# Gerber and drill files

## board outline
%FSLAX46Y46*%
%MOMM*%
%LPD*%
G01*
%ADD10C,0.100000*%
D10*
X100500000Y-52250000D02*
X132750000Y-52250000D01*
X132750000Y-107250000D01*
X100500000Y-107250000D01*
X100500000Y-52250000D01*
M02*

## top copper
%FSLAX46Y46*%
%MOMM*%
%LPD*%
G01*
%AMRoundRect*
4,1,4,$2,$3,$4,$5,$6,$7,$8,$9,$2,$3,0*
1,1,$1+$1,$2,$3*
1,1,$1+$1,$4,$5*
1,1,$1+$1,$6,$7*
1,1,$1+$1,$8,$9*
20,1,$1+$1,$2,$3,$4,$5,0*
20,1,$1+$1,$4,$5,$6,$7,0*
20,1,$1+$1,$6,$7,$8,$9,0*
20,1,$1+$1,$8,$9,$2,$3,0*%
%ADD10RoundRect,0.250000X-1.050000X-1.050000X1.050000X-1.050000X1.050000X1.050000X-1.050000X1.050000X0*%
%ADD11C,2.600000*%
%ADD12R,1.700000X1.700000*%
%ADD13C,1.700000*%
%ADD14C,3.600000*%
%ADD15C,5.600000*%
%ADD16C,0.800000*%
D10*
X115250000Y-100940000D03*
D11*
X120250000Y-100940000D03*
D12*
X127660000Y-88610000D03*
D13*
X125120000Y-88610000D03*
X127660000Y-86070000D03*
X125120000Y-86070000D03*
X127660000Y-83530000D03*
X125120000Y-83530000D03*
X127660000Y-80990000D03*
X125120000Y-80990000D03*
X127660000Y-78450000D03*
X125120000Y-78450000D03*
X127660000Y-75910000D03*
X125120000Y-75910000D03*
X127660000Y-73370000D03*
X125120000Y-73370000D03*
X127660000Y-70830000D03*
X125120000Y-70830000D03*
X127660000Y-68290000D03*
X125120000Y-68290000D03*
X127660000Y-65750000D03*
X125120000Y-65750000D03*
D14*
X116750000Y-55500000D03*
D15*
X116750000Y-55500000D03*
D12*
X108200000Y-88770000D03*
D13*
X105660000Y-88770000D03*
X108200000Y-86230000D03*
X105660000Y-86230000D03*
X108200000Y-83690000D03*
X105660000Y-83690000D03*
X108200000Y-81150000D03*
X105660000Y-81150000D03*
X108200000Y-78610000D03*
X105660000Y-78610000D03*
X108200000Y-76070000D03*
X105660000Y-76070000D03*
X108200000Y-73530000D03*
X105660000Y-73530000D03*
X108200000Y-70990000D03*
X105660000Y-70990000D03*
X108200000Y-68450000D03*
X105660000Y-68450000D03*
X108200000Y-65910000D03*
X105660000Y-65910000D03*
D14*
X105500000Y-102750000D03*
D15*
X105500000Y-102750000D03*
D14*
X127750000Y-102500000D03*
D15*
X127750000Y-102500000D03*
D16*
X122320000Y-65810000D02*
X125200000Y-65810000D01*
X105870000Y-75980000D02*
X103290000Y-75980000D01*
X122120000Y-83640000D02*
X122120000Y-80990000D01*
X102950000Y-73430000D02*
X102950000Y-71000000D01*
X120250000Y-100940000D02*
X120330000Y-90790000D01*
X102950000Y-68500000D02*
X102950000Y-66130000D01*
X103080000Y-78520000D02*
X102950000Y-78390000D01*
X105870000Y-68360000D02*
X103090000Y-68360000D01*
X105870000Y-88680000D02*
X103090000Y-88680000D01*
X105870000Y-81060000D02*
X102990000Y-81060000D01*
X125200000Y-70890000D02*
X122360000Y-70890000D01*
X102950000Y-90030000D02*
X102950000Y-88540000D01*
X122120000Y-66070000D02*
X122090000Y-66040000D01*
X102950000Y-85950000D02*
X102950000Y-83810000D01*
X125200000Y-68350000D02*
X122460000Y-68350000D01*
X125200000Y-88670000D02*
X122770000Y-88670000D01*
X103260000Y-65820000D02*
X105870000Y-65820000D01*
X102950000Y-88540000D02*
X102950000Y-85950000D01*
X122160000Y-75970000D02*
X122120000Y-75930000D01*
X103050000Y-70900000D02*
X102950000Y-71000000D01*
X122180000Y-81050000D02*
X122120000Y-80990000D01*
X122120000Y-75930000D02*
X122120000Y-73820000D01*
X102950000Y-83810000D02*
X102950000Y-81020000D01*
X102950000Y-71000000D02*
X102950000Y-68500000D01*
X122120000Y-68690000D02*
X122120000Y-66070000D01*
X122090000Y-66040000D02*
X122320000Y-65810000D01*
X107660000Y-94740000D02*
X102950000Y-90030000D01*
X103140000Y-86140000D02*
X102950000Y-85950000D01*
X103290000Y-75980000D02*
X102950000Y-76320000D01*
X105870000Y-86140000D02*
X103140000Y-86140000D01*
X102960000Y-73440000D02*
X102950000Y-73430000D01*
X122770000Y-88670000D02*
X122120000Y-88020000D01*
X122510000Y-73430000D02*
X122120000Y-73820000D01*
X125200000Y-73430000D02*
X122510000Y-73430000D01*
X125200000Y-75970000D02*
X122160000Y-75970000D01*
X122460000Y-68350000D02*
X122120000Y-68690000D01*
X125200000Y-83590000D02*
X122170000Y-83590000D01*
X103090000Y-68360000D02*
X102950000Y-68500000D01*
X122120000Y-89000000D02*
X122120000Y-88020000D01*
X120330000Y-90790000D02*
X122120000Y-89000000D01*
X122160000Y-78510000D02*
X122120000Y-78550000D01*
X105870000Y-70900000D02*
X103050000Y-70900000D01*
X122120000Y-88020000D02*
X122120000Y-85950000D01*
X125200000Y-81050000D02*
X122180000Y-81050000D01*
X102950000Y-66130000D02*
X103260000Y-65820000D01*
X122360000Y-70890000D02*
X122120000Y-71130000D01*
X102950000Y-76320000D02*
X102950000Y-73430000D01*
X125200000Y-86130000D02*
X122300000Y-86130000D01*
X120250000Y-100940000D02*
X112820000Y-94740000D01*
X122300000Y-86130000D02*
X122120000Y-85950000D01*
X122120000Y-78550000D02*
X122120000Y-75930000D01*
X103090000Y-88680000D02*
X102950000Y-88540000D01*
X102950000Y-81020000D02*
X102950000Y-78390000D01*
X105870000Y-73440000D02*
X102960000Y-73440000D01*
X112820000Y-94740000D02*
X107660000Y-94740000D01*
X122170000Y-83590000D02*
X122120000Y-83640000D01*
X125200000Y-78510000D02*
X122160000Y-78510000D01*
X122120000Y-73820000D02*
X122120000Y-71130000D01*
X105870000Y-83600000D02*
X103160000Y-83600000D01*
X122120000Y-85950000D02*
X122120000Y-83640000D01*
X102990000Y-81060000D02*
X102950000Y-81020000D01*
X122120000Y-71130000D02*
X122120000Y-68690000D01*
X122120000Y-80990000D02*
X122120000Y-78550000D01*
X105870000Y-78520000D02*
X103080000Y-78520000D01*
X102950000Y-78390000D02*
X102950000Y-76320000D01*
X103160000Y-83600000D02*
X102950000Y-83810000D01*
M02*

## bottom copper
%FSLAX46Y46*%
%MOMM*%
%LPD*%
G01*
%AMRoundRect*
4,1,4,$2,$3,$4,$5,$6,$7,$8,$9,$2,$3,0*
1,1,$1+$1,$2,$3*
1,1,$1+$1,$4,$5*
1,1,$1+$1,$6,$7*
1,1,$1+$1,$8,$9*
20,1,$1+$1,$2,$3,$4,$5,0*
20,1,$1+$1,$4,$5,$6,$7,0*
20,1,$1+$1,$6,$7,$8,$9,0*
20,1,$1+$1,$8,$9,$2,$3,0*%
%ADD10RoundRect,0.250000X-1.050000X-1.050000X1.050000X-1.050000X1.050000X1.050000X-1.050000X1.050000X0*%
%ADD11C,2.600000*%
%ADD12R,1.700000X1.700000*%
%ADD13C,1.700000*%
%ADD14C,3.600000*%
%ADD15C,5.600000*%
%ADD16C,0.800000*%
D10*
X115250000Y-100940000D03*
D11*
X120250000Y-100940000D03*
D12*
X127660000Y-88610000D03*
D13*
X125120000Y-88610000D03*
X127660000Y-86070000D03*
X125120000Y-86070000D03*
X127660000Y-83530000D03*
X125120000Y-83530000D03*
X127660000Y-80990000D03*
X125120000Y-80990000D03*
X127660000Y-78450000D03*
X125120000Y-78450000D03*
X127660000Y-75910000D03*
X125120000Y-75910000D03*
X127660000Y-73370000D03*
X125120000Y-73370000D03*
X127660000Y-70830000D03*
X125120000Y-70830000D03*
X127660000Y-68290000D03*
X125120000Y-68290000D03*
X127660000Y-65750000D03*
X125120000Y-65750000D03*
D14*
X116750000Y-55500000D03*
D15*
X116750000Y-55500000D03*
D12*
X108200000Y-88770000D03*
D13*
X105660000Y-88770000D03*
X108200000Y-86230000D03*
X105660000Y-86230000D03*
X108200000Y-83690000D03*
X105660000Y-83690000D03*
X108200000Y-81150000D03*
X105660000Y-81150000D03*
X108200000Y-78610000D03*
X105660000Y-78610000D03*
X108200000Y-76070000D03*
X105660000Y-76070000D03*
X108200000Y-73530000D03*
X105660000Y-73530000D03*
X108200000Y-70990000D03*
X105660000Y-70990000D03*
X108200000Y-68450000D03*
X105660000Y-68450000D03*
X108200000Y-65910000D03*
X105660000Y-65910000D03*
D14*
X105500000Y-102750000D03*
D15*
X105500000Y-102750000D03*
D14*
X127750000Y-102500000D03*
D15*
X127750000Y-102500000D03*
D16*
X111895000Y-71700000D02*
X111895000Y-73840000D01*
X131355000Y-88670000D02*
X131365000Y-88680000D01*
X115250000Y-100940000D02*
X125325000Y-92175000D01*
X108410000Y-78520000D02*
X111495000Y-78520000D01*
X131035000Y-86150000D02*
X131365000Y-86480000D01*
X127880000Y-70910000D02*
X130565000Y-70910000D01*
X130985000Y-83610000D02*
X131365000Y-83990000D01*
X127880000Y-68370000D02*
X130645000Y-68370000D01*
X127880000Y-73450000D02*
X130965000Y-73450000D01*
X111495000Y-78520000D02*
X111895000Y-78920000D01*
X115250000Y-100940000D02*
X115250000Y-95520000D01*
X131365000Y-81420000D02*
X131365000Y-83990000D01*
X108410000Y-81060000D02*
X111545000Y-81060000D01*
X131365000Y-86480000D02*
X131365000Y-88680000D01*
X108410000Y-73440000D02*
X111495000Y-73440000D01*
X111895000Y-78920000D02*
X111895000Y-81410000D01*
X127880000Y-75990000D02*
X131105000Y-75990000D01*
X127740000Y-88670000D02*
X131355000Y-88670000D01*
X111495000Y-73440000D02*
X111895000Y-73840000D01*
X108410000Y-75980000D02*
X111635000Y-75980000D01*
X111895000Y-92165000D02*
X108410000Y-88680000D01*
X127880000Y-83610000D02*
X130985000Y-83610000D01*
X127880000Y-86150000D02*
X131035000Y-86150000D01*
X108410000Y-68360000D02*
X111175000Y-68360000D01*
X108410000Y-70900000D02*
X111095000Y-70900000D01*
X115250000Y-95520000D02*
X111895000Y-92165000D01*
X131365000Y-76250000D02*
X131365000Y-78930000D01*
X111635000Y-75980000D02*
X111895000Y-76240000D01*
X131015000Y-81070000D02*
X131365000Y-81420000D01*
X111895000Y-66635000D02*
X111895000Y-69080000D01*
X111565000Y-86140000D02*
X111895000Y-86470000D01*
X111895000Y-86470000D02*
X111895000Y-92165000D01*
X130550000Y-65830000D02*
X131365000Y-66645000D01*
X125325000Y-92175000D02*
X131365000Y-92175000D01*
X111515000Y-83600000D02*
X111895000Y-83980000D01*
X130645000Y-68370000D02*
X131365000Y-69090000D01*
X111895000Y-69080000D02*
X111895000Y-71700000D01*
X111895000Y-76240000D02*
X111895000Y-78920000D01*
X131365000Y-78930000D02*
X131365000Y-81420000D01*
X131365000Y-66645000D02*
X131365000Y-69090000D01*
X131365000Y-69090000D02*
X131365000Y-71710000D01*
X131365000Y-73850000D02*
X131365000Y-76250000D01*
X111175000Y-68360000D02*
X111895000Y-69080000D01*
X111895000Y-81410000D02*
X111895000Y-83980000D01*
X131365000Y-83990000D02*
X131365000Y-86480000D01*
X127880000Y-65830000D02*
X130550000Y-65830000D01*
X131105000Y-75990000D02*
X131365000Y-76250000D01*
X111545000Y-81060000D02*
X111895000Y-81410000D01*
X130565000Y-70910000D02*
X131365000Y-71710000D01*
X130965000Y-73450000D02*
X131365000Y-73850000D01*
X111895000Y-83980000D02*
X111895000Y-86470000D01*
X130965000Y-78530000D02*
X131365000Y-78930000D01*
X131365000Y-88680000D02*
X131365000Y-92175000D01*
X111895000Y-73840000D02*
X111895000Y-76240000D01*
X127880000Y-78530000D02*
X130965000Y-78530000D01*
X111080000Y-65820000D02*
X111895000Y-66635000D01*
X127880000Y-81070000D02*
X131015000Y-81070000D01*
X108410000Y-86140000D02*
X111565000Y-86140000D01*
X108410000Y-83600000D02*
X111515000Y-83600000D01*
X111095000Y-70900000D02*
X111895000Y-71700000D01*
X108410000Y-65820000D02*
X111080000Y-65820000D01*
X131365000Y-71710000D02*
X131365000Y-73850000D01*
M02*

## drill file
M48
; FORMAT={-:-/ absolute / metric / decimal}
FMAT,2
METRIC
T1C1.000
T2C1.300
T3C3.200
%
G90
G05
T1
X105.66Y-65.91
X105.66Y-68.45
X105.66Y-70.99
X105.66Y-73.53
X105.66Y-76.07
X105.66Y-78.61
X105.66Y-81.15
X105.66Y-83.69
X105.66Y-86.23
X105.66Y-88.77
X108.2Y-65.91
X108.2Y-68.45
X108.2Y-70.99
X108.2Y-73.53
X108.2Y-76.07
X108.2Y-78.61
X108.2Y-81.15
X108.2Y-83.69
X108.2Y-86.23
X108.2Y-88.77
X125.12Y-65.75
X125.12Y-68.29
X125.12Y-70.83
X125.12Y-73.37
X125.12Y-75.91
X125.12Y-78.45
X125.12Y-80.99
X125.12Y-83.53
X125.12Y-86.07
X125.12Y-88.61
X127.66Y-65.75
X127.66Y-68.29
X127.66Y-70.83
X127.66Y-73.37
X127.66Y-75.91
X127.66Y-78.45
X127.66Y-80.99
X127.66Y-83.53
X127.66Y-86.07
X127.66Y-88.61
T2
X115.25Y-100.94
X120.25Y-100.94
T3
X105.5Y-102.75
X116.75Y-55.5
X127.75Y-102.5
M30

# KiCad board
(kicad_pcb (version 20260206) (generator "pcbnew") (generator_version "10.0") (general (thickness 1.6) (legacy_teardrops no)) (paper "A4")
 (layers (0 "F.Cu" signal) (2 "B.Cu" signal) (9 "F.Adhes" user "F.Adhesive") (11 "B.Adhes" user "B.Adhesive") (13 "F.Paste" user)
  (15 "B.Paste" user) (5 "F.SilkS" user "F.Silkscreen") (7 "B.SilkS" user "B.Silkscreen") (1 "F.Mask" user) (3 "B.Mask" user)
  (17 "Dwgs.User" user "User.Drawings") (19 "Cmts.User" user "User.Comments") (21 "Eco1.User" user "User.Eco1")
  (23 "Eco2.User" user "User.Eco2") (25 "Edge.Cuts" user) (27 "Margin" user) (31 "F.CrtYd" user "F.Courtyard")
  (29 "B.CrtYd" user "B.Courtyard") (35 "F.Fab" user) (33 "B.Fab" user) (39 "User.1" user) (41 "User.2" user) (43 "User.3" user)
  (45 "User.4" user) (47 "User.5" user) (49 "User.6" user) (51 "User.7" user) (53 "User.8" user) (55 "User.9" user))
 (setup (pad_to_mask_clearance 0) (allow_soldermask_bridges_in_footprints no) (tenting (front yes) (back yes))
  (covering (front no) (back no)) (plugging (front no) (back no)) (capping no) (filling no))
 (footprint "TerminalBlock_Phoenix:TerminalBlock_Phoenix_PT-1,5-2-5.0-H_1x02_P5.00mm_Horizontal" (layer "F.Cu") (at 115.25 100.94)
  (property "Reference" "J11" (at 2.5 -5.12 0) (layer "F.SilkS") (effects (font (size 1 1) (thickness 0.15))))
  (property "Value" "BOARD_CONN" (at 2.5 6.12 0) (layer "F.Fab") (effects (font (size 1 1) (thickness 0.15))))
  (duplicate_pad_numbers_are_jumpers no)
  (pad "1" thru_hole roundrect (at 0 0) (size 2.6 2.6) (drill 1.3) (layers "*.Cu" "*.Mask") (remove_unused_layers no)
   (roundrect_rratio 0.096154) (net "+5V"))
  (pad "2" thru_hole circle (at 5 0) (size 2.6 2.6) (drill 1.3) (layers "*.Cu" "*.Mask") (remove_unused_layers no) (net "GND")))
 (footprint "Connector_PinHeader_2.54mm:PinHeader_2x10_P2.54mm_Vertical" (layer "F.Cu") (at 127.66 88.61 180)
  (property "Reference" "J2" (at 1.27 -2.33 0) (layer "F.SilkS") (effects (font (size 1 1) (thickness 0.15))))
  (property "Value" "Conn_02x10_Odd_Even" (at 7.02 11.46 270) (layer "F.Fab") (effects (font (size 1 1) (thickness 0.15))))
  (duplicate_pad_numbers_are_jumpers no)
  (pad "1" thru_hole rect (at 0 0 180) (size 1.7 1.7) (drill 1) (layers "*.Cu" "*.Mask") (remove_unused_layers no) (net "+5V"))
  (pad "2" thru_hole circle (at 2.54 0 180) (size 1.7 1.7) (drill 1) (layers "*.Cu" "*.Mask") (remove_unused_layers no) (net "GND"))
  (pad "3" thru_hole circle (at 0 2.54 180) (size 1.7 1.7) (drill 1) (layers "*.Cu" "*.Mask") (remove_unused_layers no) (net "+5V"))
  (pad "4" thru_hole circle (at 2.54 2.54 180) (size 1.7 1.7) (drill 1) (layers "*.Cu" "*.Mask") (remove_unused_layers no) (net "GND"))
  (pad "5" thru_hole circle (at 0 5.08 180) (size 1.7 1.7) (drill 1) (layers "*.Cu" "*.Mask") (remove_unused_layers no) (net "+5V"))
  (pad "6" thru_hole circle (at 2.54 5.08 180) (size 1.7 1.7) (drill 1) (layers "*.Cu" "*.Mask") (remove_unused_layers no) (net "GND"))
  (pad "7" thru_hole circle (at 0 7.62 180) (size 1.7 1.7) (drill 1) (layers "*.Cu" "*.Mask") (remove_unused_layers no) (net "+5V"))
  (pad "8" thru_hole circle (at 2.54 7.62 180) (size 1.7 1.7) (drill 1) (layers "*.Cu" "*.Mask") (remove_unused_layers no) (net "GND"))
  (pad "9" thru_hole circle (at 0 10.16 180) (size 1.7 1.7) (drill 1) (layers "*.Cu" "*.Mask") (remove_unused_layers no) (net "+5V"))
  (pad "10" thru_hole circle (at 2.54 10.16 180) (size 1.7 1.7) (drill 1) (layers "*.Cu" "*.Mask") (remove_unused_layers no) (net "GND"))
  (pad "11" thru_hole circle (at 0 12.7 180) (size 1.7 1.7) (drill 1) (layers "*.Cu" "*.Mask") (remove_unused_layers no) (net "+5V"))
  (pad "12" thru_hole circle (at 2.54 12.7 180) (size 1.7 1.7) (drill 1) (layers "*.Cu" "*.Mask") (remove_unused_layers no) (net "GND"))
  (pad "13" thru_hole circle (at 0 15.24 180) (size 1.7 1.7) (drill 1) (layers "*.Cu" "*.Mask") (remove_unused_layers no) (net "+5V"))
  (pad "14" thru_hole circle (at 2.54 15.24 180) (size 1.7 1.7) (drill 1) (layers "*.Cu" "*.Mask") (remove_unused_layers no) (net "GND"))
  (pad "15" thru_hole circle (at 0 17.78 180) (size 1.7 1.7) (drill 1) (layers "*.Cu" "*.Mask") (remove_unused_layers no) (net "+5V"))
  (pad "16" thru_hole circle (at 2.54 17.78 180) (size 1.7 1.7) (drill 1) (layers "*.Cu" "*.Mask") (remove_unused_layers no) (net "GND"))
  (pad "17" thru_hole circle (at 0 20.32 180) (size 1.7 1.7) (drill 1) (layers "*.Cu" "*.Mask") (remove_unused_layers no) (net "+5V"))
  (pad "18" thru_hole circle (at 2.54 20.32 180) (size 1.7 1.7) (drill 1) (layers "*.Cu" "*.Mask") (remove_unused_layers no) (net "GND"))
  (pad "19" thru_hole circle (at 0 22.86 180) (size 1.7 1.7) (drill 1) (layers "*.Cu" "*.Mask") (remove_unused_layers no) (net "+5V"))
  (pad "20" thru_hole circle (at 2.54 22.86 180) (size 1.7 1.7) (drill 1) (layers "*.Cu" "*.Mask") (remove_unused_layers no) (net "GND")))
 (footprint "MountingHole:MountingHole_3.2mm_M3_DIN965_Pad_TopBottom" (layer "F.Cu") (at 116.75 55.5)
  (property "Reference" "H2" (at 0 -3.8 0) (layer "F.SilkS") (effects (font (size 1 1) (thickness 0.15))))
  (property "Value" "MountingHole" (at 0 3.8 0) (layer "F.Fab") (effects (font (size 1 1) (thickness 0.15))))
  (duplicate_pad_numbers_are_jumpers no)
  (pad "1" thru_hole circle (at 0 0) (size 3.6 3.6) (drill 3.2) (layers "*.Cu" "*.Mask") (remove_unused_layers no) (zone_connect 2))
  (pad "1" connect circle (at 0 0) (size 5.6 5.6) (layers "F.Cu" "F.Mask") (zone_connect 2))
  (pad "1" connect circle (at 0 0) (size 5.6 5.6) (layers "B.Cu" "B.Mask") (zone_connect 2)))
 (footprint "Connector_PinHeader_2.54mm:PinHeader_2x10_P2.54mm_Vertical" (layer "F.Cu") (at 108.2 88.77 180)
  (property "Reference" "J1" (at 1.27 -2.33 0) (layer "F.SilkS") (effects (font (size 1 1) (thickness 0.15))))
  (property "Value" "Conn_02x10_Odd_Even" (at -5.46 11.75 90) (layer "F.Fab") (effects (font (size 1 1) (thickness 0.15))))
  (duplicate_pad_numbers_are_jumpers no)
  (pad "1" thru_hole rect (at 0 0 180) (size 1.7 1.7) (drill 1) (layers "*.Cu" "*.Mask") (remove_unused_layers no) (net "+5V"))
  (pad "2" thru_hole circle (at 2.54 0 180) (size 1.7 1.7) (drill 1) (layers "*.Cu" "*.Mask") (remove_unused_layers no) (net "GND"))
  (pad "3" thru_hole circle (at 0 2.54 180) (size 1.7 1.7) (drill 1) (layers "*.Cu" "*.Mask") (remove_unused_layers no) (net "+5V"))
  (pad "4" thru_hole circle (at 2.54 2.54 180) (size 1.7 1.7) (drill 1) (layers "*.Cu" "*.Mask") (remove_unused_layers no) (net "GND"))
  (pad "5" thru_hole circle (at 0 5.08 180) (size 1.7 1.7) (drill 1) (layers "*.Cu" "*.Mask") (remove_unused_layers no) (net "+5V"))
  (pad "6" thru_hole circle (at 2.54 5.08 180) (size 1.7 1.7) (drill 1) (layers "*.Cu" "*.Mask") (remove_unused_layers no) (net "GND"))
  (pad "7" thru_hole circle (at 0 7.62 180) (size 1.7 1.7) (drill 1) (layers "*.Cu" "*.Mask") (remove_unused_layers no) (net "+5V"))
  (pad "8" thru_hole circle (at 2.54 7.62 180) (size 1.7 1.7) (drill 1) (layers "*.Cu" "*.Mask") (remove_unused_layers no) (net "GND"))
  (pad "9" thru_hole circle (at 0 10.16 180) (size 1.7 1.7) (drill 1) (layers "*.Cu" "*.Mask") (remove_unused_layers no) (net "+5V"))
  (pad "10" thru_hole circle (at 2.54 10.16 180) (size 1.7 1.7) (drill 1) (layers "*.Cu" "*.Mask") (remove_unused_layers no) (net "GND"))
  (pad "11" thru_hole circle (at 0 12.7 180) (size 1.7 1.7) (drill 1) (layers "*.Cu" "*.Mask") (remove_unused_layers no) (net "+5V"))
  (pad "12" thru_hole circle (at 2.54 12.7 180) (size 1.7 1.7) (drill 1) (layers "*.Cu" "*.Mask") (remove_unused_layers no) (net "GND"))
  (pad "13" thru_hole circle (at 0 15.24 180) (size 1.7 1.7) (drill 1) (layers "*.Cu" "*.Mask") (remove_unused_layers no) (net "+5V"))
  (pad "14" thru_hole circle (at 2.54 15.24 180) (size 1.7 1.7) (drill 1) (layers "*.Cu" "*.Mask") (remove_unused_layers no) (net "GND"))
  (pad "15" thru_hole circle (at 0 17.78 180) (size 1.7 1.7) (drill 1) (layers "*.Cu" "*.Mask") (remove_unused_layers no) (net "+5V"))
  (pad "16" thru_hole circle (at 2.54 17.78 180) (size 1.7 1.7) (drill 1) (layers "*.Cu" "*.Mask") (remove_unused_layers no) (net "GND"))
  (pad "17" thru_hole circle (at 0 20.32 180) (size 1.7 1.7) (drill 1) (layers "*.Cu" "*.Mask") (remove_unused_layers no) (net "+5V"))
  (pad "18" thru_hole circle (at 2.54 20.32 180) (size 1.7 1.7) (drill 1) (layers "*.Cu" "*.Mask") (remove_unused_layers no) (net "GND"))
  (pad "19" thru_hole circle (at 0 22.86 180) (size 1.7 1.7) (drill 1) (layers "*.Cu" "*.Mask") (remove_unused_layers no) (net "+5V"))
  (pad "20" thru_hole circle (at 2.54 22.86 180) (size 1.7 1.7) (drill 1) (layers "*.Cu" "*.Mask") (remove_unused_layers no) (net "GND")))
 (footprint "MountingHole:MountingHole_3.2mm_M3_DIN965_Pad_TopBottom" (layer "F.Cu") (at 105.5 102.75)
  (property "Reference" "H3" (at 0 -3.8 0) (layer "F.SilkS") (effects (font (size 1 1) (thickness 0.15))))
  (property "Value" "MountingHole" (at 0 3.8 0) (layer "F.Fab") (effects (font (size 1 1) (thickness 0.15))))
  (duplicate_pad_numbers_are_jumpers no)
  (pad "1" thru_hole circle (at 0 0) (size 3.6 3.6) (drill 3.2) (layers "*.Cu" "*.Mask") (remove_unused_layers no) (zone_connect 2))
  (pad "1" connect circle (at 0 0) (size 5.6 5.6) (layers "F.Cu" "F.Mask") (zone_connect 2))
  (pad "1" connect circle (at 0 0) (size 5.6 5.6) (layers "B.Cu" "B.Mask") (zone_connect 2)))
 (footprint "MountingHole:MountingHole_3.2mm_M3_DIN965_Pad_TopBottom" (layer "F.Cu") (at 127.75 102.5)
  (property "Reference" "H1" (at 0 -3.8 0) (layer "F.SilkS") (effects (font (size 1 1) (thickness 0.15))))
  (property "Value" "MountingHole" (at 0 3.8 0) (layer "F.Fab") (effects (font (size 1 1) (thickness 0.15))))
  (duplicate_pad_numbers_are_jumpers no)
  (pad "1" thru_hole circle (at 0 0) (size 3.6 3.6) (drill 3.2) (layers "*.Cu" "*.Mask") (remove_unused_layers no) (zone_connect 2))
  (pad "1" connect circle (at 0 0) (size 5.6 5.6) (layers "F.Cu" "F.Mask") (zone_connect 2))
  (pad "1" connect circle (at 0 0) (size 5.6 5.6) (layers "B.Cu" "B.Mask") (zone_connect 2)))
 (gr_rect (start 100.5 52.25) (end 132.75 107.25) (stroke (width 0.1) (type default)) (fill no) (layer "Edge.Cuts"))
 (segment (start 111.895 71.7) (end 111.895 73.84) (width 0.8) (layer "B.Cu") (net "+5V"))
 (segment (start 131.355 88.67) (end 131.365 88.68) (width 0.8) (layer "B.Cu") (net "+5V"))
 (segment (start 115.25 100.94) (end 125.325 92.175) (width 0.8) (layer "B.Cu") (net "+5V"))
 (segment (start 108.41 78.52) (end 111.495 78.52) (width 0.8) (layer "B.Cu") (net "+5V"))
 (segment (start 131.035 86.15) (end 131.365 86.48) (width 0.8) (layer "B.Cu") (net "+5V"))
 (segment (start 127.88 70.91) (end 130.565 70.91) (width 0.8) (layer "B.Cu") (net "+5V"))
 (segment (start 130.985 83.61) (end 131.365 83.99) (width 0.8) (layer "B.Cu") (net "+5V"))
 (segment (start 127.88 68.37) (end 130.645 68.37) (width 0.8) (layer "B.Cu") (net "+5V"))
 (segment (start 127.88 73.45) (end 130.965 73.45) (width 0.8) (layer "B.Cu") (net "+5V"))
 (segment (start 111.495 78.52) (end 111.895 78.92) (width 0.8) (layer "B.Cu") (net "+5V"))
 (segment (start 115.25 100.94) (end 115.25 95.52) (width 0.8) (layer "B.Cu") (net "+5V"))
 (segment (start 131.365 81.42) (end 131.365 83.99) (width 0.8) (layer "B.Cu") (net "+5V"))
 (segment (start 108.41 81.06) (end 111.545 81.06) (width 0.8) (layer "B.Cu") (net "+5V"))
 (segment (start 131.365 86.48) (end 131.365 88.68) (width 0.8) (layer "B.Cu") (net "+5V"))
 (segment (start 108.41 73.44) (end 111.495 73.44) (width 0.8) (layer "B.Cu") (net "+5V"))
 (segment (start 111.895 78.92) (end 111.895 81.41) (width 0.8) (layer "B.Cu") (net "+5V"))
 (segment (start 127.88 75.99) (end 131.105 75.99) (width 0.8) (layer "B.Cu") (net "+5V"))
 (segment (start 127.74 88.67) (end 131.355 88.67) (width 0.8) (layer "B.Cu") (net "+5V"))
 (segment (start 111.495 73.44) (end 111.895 73.84) (width 0.8) (layer "B.Cu") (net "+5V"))
 (segment (start 108.41 75.98) (end 111.635 75.98) (width 0.8) (layer "B.Cu") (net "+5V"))
 (segment (start 111.895 92.165) (end 108.41 88.68) (width 0.8) (layer "B.Cu") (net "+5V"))
 (segment (start 127.88 83.61) (end 130.985 83.61) (width 0.8) (layer "B.Cu") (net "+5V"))
 (segment (start 127.88 86.15) (end 131.035 86.15) (width 0.8) (layer "B.Cu") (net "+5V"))
 (segment (start 108.41 68.36) (end 111.175 68.36) (width 0.8) (layer "B.Cu") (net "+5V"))
 (segment (start 108.41 70.9) (end 111.095 70.9) (width 0.8) (layer "B.Cu") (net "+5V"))
 (segment (start 115.25 95.52) (end 111.895 92.165) (width 0.8) (layer "B.Cu") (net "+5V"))
 (segment (start 131.365 76.25) (end 131.365 78.93) (width 0.8) (layer "B.Cu") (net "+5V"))
 (segment (start 111.635 75.98) (end 111.895 76.24) (width 0.8) (layer "B.Cu") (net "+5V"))
 (segment (start 131.015 81.07) (end 131.365 81.42) (width 0.8) (layer "B.Cu") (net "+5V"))
 (segment (start 111.895 66.635) (end 111.895 69.08) (width 0.8) (layer "B.Cu") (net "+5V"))
 (segment (start 111.565 86.14) (end 111.895 86.47) (width 0.8) (layer "B.Cu") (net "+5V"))
 (segment (start 111.895 86.47) (end 111.895 92.165) (width 0.8) (layer "B.Cu") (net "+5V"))
 (segment (start 130.55 65.83) (end 131.365 66.645) (width 0.8) (layer "B.Cu") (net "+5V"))
 (segment (start 125.325 92.175) (end 131.365 92.175) (width 0.8) (layer "B.Cu") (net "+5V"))
 (segment (start 111.515 83.6) (end 111.895 83.98) (width 0.8) (layer "B.Cu") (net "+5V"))
 (segment (start 130.645 68.37) (end 131.365 69.09) (width 0.8) (layer "B.Cu") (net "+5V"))
 (segment (start 111.895 69.08) (end 111.895 71.7) (width 0.8) (layer "B.Cu") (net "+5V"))
 (segment (start 111.895 76.24) (end 111.895 78.92) (width 0.8) (layer "B.Cu") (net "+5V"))
 (segment (start 131.365 78.93) (end 131.365 81.42) (width 0.8) (layer "B.Cu") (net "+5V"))
 (segment (start 131.365 66.645) (end 131.365 69.09) (width 0.8) (layer "B.Cu") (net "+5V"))
 (segment (start 131.365 69.09) (end 131.365 71.71) (width 0.8) (layer "B.Cu") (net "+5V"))
 (segment (start 131.365 73.85) (end 131.365 76.25) (width 0.8) (layer "B.Cu") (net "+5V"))
 (segment (start 111.175 68.36) (end 111.895 69.08) (width 0.8) (layer "B.Cu") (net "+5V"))
 (segment (start 111.895 81.41) (end 111.895 83.98) (width 0.8) (layer "B.Cu") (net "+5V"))
 (segment (start 131.365 83.99) (end 131.365 86.48) (width 0.8) (layer "B.Cu") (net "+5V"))
 (segment (start 127.88 65.83) (end 130.55 65.83) (width 0.8) (layer "B.Cu") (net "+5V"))
 (segment (start 131.105 75.99) (end 131.365 76.25) (width 0.8) (layer "B.Cu") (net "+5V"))
 (segment (start 111.545 81.06) (end 111.895 81.41) (width 0.8) (layer "B.Cu") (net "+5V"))
 (segment (start 130.565 70.91) (end 131.365 71.71) (width 0.8) (layer "B.Cu") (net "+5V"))
 (segment (start 130.965 73.45) (end 131.365 73.85) (width 0.8) (layer "B.Cu") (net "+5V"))
 (segment (start 111.895 83.98) (end 111.895 86.47) (width 0.8) (layer "B.Cu") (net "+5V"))
 (segment (start 130.965 78.53) (end 131.365 78.93) (width 0.8) (layer "B.Cu") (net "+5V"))
 (segment (start 131.365 88.68) (end 131.365 92.175) (width 0.8) (layer "B.Cu") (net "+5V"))
 (segment (start 111.895 73.84) (end 111.895 76.24) (width 0.8) (layer "B.Cu") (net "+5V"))
 (segment (start 127.88 78.53) (end 130.965 78.53) (width 0.8) (layer "B.Cu") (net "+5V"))
 (segment (start 111.08 65.82) (end 111.895 66.635) (width 0.8) (layer "B.Cu") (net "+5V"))
 (segment (start 127.88 81.07) (end 131.015 81.07) (width 0.8) (layer "B.Cu") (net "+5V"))
 (segment (start 108.41 86.14) (end 111.565 86.14) (width 0.8) (layer "B.Cu") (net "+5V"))
 (segment (start 108.41 83.6) (end 111.515 83.6) (width 0.8) (layer "B.Cu") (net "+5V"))
 (segment (start 111.095 70.9) (end 111.895 71.7) (width 0.8) (layer "B.Cu") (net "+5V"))
 (segment (start 108.41 65.82) (end 111.08 65.82) (width 0.8) (layer "B.Cu") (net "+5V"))
 (segment (start 131.365 71.71) (end 131.365 73.85) (width 0.8) (layer "B.Cu") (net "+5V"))
 (segment (start 122.32 65.81) (end 125.2 65.81) (width 0.8) (layer "F.Cu") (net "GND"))
 (segment (start 105.87 75.98) (end 103.29 75.98) (width 0.8) (layer "F.Cu") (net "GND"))
 (segment (start 122.12 83.64) (end 122.12 80.99) (width 0.8) (layer "F.Cu") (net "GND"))
 (segment (start 102.95 73.43) (end 102.95 71) (width 0.8) (layer "F.Cu") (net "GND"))
 (segment (start 120.25 100.94) (end 120.33 90.79) (width 0.8) (layer "F.Cu") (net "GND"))
 (segment (start 102.95 68.5) (end 102.95 66.13) (width 0.8) (layer "F.Cu") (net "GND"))
 (segment (start 103.08 78.52) (end 102.95 78.39) (width 0.8) (layer "F.Cu") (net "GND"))
 (segment (start 105.87 68.36) (end 103.09 68.36) (width 0.8) (layer "F.Cu") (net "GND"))
 (segment (start 105.87 88.68) (end 103.09 88.68) (width 0.8) (layer "F.Cu") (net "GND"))
 (segment (start 105.87 81.06) (end 102.99 81.06) (width 0.8) (layer "F.Cu") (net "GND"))
 (segment (start 125.2 70.89) (end 122.36 70.89) (width 0.8) (layer "F.Cu") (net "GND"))
 (segment (start 102.95 90.03) (end 102.95 88.54) (width 0.8) (layer "F.Cu") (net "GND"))
 (segment (start 122.12 66.07) (end 122.09 66.04) (width 0.8) (layer "F.Cu") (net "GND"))
 (segment (start 102.95 85.95) (end 102.95 83.81) (width 0.8) (layer "F.Cu") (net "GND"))
 (segment (start 125.2 68.35) (end 122.46 68.35) (width 0.8) (layer "F.Cu") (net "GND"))
 (segment (start 125.2 88.67) (end 122.77 88.67) (width 0.8) (layer "F.Cu") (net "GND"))
 (segment (start 103.26 65.82) (end 105.87 65.82) (width 0.8) (layer "F.Cu") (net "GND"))
 (segment (start 102.95 88.54) (end 102.95 85.95) (width 0.8) (layer "F.Cu") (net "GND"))
 (segment (start 122.16 75.97) (end 122.12 75.93) (width 0.8) (layer "F.Cu") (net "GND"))
 (segment (start 103.05 70.9) (end 102.95 71) (width 0.8) (layer "F.Cu") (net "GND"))
 (segment (start 122.18 81.05) (end 122.12 80.99) (width 0.8) (layer "F.Cu") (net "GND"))
 (segment (start 122.12 75.93) (end 122.12 73.82) (width 0.8) (layer "F.Cu") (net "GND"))
 (segment (start 102.95 83.81) (end 102.95 81.02) (width 0.8) (layer "F.Cu") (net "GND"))
 (segment (start 102.95 71) (end 102.95 68.5) (width 0.8) (layer "F.Cu") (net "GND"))
 (segment (start 122.12 68.69) (end 122.12 66.07) (width 0.8) (layer "F.Cu") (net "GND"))
 (segment (start 122.09 66.04) (end 122.32 65.81) (width 0.8) (layer "F.Cu") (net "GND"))
 (segment (start 107.66 94.74) (end 102.95 90.03) (width 0.8) (layer "F.Cu") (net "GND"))
 (segment (start 103.14 86.14) (end 102.95 85.95) (width 0.8) (layer "F.Cu") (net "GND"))
 (segment (start 103.29 75.98) (end 102.95 76.32) (width 0.8) (layer "F.Cu") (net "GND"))
 (segment (start 105.87 86.14) (end 103.14 86.14) (width 0.8) (layer "F.Cu") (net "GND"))
 (segment (start 102.96 73.44) (end 102.95 73.43) (width 0.8) (layer "F.Cu") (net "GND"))
 (segment (start 122.77 88.67) (end 122.12 88.02) (width 0.8) (layer "F.Cu") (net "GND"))
 (segment (start 122.51 73.43) (end 122.12 73.82) (width 0.8) (layer "F.Cu") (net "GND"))
 (segment (start 125.2 73.43) (end 122.51 73.43) (width 0.8) (layer "F.Cu") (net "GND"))
 (segment (start 125.2 75.97) (end 122.16 75.97) (width 0.8) (layer "F.Cu") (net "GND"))
 (segment (start 122.46 68.35) (end 122.12 68.69) (width 0.8) (layer "F.Cu") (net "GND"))
 (segment (start 125.2 83.59) (end 122.17 83.59) (width 0.8) (layer "F.Cu") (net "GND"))
 (segment (start 103.09 68.36) (end 102.95 68.5) (width 0.8) (layer "F.Cu") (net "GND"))
 (segment (start 122.12 89) (end 122.12 88.02) (width 0.8) (layer "F.Cu") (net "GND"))
 (segment (start 120.33 90.79) (end 122.12 89) (width 0.8) (layer "F.Cu") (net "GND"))
 (segment (start 122.16 78.51) (end 122.12 78.55) (width 0.8) (layer "F.Cu") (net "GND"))
 (segment (start 105.87 70.9) (end 103.05 70.9) (width 0.8) (layer "F.Cu") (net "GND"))
 (segment (start 122.12 88.02) (end 122.12 85.95) (width 0.8) (layer "F.Cu") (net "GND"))
 (segment (start 125.2 81.05) (end 122.18 81.05) (width 0.8) (layer "F.Cu") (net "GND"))
 (segment (start 102.95 66.13) (end 103.26 65.82) (width 0.8) (layer "F.Cu") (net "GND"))
 (segment (start 122.36 70.89) (end 122.12 71.13) (width 0.8) (layer "F.Cu") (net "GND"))
 (segment (start 102.95 76.32) (end 102.95 73.43) (width 0.8) (layer "F.Cu") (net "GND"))
 (segment (start 125.2 86.13) (end 122.3 86.13) (width 0.8) (layer "F.Cu") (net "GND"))
 (segment (start 120.25 100.94) (end 112.82 94.74) (width 0.8) (layer "F.Cu") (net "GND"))
 (segment (start 122.3 86.13) (end 122.12 85.95) (width 0.8) (layer "F.Cu") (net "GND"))
 (segment (start 122.12 78.55) (end 122.12 75.93) (width 0.8) (layer "F.Cu") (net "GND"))
 (segment (start 103.09 88.68) (end 102.95 88.54) (width 0.8) (layer "F.Cu") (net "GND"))
 (segment (start 102.95 81.02) (end 102.95 78.39) (width 0.8) (layer "F.Cu") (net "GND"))
 (segment (start 105.87 73.44) (end 102.96 73.44) (width 0.8) (layer "F.Cu") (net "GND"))
 (segment (start 112.82 94.74) (end 107.66 94.74) (width 0.8) (layer "F.Cu") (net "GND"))
 (segment (start 122.17 83.59) (end 122.12 83.64) (width 0.8) (layer "F.Cu") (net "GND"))
 (segment (start 125.2 78.51) (end 122.16 78.51) (width 0.8) (layer "F.Cu") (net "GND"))
 (segment (start 122.12 73.82) (end 122.12 71.13) (width 0.8) (layer "F.Cu") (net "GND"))
 (segment (start 105.87 83.6) (end 103.16 83.6) (width 0.8) (layer "F.Cu") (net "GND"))
 (segment (start 122.12 85.95) (end 122.12 83.64) (width 0.8) (layer "F.Cu") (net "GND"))
 (segment (start 102.99 81.06) (end 102.95 81.02) (width 0.8) (layer "F.Cu") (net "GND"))
 (segment (start 122.12 71.13) (end 122.12 68.69) (width 0.8) (layer "F.Cu") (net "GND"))
 (segment (start 122.12 80.99) (end 122.12 78.55) (width 0.8) (layer "F.Cu") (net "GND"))
 (segment (start 105.87 78.52) (end 103.08 78.52) (width 0.8) (layer "F.Cu") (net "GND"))
 (segment (start 102.95 78.39) (end 102.95 76.32) (width 0.8) (layer "F.Cu") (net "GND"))
 (segment (start 103.16 83.6) (end 102.95 83.81) (width 0.8) (layer "F.Cu") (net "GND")))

